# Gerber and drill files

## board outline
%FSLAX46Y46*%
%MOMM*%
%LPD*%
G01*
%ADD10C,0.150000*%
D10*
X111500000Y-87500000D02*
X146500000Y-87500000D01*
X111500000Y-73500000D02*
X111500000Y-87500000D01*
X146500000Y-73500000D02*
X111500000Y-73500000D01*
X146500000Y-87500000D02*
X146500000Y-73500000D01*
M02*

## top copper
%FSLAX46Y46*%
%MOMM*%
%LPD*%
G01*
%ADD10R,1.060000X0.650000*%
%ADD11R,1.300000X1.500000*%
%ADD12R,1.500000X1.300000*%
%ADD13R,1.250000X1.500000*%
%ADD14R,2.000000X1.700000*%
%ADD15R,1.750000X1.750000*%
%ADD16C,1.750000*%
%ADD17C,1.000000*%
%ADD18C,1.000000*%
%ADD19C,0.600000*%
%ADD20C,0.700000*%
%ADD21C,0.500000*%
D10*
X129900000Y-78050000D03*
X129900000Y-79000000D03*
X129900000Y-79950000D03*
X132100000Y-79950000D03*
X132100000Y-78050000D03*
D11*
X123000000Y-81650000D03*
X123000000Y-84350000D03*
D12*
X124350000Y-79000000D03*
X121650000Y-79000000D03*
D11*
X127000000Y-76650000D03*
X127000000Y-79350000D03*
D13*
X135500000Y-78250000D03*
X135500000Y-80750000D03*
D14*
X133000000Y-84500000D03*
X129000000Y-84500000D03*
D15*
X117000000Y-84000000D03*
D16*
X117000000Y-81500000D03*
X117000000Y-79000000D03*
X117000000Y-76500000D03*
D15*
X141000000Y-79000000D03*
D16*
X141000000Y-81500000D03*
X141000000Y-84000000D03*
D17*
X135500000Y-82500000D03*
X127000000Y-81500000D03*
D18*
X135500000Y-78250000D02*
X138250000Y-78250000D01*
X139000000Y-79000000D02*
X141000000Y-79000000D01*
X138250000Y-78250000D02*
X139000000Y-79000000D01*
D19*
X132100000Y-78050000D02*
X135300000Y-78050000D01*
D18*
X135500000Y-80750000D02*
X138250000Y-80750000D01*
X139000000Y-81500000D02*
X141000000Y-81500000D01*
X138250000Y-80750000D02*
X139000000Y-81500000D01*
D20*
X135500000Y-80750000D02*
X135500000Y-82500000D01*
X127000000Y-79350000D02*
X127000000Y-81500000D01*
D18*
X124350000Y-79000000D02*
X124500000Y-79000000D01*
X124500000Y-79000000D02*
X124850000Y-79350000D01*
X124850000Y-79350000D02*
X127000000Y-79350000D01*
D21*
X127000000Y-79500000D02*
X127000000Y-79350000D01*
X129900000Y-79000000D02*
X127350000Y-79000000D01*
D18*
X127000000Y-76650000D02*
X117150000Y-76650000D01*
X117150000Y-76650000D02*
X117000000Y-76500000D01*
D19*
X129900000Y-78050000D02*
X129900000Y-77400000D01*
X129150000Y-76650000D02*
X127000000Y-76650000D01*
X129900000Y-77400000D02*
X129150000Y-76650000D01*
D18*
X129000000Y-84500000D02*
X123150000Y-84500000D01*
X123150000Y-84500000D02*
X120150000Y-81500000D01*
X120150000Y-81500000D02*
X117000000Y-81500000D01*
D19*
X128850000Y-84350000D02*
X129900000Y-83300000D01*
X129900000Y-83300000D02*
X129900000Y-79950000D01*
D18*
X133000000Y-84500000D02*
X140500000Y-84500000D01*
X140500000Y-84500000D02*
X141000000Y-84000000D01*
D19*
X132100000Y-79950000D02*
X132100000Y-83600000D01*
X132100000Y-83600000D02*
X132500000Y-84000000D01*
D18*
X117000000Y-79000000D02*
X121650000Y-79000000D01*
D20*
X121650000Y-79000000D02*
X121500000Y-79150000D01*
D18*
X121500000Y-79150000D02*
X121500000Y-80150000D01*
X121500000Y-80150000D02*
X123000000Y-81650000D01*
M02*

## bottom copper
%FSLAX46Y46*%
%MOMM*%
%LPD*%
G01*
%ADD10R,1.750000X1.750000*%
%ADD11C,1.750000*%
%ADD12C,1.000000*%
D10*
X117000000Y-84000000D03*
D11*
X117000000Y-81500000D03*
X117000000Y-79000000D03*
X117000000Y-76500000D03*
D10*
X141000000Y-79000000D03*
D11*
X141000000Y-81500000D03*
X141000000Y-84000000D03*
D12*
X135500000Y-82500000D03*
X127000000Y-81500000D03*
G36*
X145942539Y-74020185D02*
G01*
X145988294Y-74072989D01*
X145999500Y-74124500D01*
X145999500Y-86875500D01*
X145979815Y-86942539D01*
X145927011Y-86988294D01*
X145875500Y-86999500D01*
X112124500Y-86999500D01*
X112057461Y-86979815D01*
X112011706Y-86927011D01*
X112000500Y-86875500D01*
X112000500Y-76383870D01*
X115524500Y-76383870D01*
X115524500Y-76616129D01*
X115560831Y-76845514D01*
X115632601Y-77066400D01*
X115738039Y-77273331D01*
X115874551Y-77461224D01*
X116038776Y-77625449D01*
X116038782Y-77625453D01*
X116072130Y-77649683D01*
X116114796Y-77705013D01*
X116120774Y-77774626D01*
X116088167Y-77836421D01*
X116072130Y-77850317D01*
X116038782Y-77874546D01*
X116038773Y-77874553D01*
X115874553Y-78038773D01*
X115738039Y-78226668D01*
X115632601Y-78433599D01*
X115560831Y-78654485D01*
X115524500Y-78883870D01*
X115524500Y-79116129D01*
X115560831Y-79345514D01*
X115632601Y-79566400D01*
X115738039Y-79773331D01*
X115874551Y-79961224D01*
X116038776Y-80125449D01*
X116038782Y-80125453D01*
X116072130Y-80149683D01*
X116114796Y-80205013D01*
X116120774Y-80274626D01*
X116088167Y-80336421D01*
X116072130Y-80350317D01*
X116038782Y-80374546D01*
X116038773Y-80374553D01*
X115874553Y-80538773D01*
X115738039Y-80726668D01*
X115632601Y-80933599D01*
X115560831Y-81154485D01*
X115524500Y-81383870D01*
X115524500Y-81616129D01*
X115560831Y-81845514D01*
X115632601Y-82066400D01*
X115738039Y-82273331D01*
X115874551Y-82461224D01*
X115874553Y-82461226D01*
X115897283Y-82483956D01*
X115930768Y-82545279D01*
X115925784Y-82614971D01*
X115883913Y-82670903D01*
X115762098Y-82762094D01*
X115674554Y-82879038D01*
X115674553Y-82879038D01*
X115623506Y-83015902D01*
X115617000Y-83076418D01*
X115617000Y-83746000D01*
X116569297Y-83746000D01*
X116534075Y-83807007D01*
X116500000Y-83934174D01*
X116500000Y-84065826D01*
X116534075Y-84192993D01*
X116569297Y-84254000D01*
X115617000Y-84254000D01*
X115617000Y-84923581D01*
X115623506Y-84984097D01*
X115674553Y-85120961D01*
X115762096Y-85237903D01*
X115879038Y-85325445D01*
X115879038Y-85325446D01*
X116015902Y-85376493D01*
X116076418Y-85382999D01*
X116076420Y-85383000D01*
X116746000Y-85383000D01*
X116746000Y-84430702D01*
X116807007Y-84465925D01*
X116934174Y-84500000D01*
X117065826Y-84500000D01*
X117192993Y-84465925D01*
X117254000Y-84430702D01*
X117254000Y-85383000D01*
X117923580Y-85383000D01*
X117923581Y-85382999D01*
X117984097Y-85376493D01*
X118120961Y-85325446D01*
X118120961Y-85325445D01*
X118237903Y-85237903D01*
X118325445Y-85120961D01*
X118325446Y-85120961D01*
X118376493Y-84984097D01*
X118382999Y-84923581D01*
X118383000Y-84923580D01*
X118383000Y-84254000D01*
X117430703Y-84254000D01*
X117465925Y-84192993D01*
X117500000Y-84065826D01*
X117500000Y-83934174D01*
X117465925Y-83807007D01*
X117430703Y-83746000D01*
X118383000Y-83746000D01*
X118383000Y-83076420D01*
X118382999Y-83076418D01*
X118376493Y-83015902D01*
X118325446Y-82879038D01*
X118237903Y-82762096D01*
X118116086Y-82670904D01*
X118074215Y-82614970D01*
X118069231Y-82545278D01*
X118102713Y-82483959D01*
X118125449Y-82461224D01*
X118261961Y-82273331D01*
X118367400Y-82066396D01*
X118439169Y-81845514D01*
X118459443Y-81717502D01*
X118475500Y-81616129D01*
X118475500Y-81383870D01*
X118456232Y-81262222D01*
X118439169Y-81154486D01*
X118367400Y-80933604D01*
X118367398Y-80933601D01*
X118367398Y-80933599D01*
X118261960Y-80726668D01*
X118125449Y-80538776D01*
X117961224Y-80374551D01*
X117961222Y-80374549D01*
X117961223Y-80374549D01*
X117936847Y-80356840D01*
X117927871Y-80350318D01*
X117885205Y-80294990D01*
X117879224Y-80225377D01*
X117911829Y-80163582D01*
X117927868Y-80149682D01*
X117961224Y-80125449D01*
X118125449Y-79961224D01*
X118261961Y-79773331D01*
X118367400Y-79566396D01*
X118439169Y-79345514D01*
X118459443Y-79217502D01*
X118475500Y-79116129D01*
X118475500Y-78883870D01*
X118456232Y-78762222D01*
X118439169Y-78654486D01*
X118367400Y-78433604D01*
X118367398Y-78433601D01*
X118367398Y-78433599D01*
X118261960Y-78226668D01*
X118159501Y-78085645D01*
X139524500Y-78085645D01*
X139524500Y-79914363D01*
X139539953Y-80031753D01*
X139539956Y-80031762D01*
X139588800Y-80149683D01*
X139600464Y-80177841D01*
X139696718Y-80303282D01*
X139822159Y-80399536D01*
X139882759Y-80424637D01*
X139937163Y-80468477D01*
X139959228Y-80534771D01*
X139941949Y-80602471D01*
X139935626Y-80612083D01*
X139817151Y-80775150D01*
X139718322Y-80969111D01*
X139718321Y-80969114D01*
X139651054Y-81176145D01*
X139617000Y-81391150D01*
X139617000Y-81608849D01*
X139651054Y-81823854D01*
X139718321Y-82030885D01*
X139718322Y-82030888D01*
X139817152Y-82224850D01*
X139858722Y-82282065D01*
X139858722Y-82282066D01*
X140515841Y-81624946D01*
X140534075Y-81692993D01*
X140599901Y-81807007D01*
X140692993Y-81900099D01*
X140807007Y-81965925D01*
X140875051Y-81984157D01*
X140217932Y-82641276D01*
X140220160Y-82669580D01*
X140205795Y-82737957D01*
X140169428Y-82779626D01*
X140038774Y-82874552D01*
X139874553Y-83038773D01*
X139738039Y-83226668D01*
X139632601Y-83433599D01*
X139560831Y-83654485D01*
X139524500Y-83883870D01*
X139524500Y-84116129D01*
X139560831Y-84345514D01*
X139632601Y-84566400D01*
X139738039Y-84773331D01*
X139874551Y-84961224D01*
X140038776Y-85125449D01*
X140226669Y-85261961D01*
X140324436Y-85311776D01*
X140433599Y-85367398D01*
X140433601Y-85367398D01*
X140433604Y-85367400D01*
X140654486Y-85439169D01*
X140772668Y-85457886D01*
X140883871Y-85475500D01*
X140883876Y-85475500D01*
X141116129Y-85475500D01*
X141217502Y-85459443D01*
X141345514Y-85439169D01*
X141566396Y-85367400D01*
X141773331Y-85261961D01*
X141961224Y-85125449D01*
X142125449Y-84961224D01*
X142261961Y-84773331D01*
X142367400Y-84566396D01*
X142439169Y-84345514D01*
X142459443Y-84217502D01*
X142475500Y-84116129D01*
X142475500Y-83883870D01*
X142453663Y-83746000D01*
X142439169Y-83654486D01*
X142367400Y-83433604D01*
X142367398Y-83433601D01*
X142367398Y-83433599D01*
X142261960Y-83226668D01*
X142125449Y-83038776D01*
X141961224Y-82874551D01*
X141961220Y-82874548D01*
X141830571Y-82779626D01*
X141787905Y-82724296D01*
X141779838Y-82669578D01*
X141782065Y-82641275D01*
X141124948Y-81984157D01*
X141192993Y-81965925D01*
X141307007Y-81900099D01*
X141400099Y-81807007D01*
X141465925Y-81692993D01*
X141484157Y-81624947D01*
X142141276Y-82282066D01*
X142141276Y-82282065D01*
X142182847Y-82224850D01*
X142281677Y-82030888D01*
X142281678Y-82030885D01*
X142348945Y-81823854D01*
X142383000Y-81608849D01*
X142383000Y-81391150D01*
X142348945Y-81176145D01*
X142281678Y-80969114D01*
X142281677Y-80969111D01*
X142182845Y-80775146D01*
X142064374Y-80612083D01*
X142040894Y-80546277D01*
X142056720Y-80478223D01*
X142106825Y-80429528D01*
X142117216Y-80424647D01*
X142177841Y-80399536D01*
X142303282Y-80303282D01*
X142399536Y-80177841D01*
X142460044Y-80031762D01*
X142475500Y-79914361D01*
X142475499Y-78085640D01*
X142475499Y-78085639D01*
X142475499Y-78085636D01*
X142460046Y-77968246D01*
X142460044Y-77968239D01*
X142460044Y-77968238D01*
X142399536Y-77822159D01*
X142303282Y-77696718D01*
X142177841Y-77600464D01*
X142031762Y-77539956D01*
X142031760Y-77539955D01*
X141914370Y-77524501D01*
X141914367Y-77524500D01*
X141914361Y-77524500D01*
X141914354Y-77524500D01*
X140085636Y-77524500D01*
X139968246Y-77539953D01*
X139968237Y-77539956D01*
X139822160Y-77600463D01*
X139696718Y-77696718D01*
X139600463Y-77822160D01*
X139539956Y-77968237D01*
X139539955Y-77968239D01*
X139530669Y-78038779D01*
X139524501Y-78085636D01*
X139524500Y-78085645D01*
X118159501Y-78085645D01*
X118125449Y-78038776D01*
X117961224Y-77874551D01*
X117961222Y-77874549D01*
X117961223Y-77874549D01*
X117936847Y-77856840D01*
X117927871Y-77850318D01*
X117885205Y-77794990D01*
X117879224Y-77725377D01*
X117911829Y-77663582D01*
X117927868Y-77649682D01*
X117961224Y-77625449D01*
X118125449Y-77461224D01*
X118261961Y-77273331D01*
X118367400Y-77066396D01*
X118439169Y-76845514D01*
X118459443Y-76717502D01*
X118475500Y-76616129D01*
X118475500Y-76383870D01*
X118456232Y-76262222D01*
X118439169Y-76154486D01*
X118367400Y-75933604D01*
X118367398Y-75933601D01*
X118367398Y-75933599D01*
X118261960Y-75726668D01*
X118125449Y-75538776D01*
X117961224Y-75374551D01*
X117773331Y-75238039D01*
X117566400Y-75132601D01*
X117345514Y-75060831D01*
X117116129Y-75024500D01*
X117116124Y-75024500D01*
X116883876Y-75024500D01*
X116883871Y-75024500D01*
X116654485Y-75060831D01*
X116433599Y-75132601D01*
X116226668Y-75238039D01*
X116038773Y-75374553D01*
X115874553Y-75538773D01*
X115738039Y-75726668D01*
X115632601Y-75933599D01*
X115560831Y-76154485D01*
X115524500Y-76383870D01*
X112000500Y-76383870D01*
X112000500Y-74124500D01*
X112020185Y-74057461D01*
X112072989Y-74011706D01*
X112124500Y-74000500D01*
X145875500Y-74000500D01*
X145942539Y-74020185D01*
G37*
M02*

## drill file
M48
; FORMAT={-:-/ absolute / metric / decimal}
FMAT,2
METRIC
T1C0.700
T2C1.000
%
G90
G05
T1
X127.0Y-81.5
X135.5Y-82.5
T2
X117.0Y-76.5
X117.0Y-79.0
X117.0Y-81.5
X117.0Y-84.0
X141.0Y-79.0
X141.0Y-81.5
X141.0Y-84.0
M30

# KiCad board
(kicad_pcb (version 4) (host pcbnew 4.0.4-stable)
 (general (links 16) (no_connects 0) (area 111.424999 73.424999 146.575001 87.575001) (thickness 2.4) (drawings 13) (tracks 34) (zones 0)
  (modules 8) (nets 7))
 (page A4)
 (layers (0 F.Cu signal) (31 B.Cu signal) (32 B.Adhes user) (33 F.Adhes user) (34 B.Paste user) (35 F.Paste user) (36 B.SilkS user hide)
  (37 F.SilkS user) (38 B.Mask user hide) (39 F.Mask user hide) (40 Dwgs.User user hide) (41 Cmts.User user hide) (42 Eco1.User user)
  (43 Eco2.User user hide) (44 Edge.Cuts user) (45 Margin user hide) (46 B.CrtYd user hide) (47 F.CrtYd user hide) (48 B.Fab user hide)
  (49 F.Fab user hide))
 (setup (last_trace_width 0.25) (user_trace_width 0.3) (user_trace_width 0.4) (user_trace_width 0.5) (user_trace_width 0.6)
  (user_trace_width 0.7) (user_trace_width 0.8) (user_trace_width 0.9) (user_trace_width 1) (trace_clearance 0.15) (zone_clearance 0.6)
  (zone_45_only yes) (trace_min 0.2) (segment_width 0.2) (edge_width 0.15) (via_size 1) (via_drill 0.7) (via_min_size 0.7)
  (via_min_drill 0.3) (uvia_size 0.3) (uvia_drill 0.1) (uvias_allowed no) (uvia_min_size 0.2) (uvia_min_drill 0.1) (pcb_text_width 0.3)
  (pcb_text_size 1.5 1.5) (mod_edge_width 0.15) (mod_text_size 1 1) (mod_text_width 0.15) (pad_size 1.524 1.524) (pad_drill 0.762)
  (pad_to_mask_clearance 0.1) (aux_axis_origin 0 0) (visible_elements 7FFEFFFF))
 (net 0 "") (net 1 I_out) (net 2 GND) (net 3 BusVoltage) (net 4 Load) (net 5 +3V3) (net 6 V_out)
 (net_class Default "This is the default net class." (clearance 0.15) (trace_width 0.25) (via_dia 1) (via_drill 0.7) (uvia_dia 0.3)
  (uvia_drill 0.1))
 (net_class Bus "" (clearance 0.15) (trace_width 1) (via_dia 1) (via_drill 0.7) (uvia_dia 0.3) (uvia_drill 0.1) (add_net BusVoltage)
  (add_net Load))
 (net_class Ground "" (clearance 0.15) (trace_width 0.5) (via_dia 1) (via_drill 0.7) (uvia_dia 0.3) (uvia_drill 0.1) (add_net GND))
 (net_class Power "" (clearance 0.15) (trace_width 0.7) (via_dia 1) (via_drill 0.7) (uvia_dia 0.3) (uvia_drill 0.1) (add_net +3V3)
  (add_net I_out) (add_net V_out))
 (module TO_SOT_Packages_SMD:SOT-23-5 (layer F.Cu) (at 131 79)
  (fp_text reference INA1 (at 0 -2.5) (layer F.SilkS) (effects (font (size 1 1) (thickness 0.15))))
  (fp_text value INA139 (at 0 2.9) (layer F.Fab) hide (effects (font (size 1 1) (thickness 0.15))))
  (pad 1 smd rect (at -1.1 -0.95) (size 1.06 0.65) (layers F.Cu F.Paste F.Mask) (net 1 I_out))
  (pad 2 smd rect (at -1.1 0) (size 1.06 0.65) (layers F.Cu F.Paste F.Mask) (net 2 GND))
  (pad 3 smd rect (at -1.1 0.95) (size 1.06 0.65) (layers F.Cu F.Paste F.Mask) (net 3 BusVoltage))
  (pad 4 smd rect (at 1.1 0.95) (size 1.06 0.65) (layers F.Cu F.Paste F.Mask) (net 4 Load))
  (pad 5 smd rect (at 1.1 -0.95) (size 1.06 0.65) (layers F.Cu F.Paste F.Mask) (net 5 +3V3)))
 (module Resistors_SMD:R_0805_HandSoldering (layer F.Cu) (at 123 83 270)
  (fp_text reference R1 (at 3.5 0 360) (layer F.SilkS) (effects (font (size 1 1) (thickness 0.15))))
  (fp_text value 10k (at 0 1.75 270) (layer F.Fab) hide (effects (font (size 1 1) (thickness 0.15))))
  (pad 1 smd rect (at -1.35 0 270) (size 1.5 1.3) (layers F.Cu F.Paste F.Mask) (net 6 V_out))
  (pad 2 smd rect (at 1.35 0 270) (size 1.5 1.3) (layers F.Cu F.Paste F.Mask) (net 3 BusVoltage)))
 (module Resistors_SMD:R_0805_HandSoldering (layer F.Cu) (at 123 79 180)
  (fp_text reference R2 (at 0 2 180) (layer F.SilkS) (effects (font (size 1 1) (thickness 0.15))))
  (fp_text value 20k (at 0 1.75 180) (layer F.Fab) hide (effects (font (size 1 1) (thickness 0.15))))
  (pad 1 smd rect (at -1.35 0 180) (size 1.5 1.3) (layers F.Cu F.Paste F.Mask) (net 2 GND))
  (pad 2 smd rect (at 1.35 0 180) (size 1.5 1.3) (layers F.Cu F.Paste F.Mask) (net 6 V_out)))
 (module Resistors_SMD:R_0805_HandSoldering (layer F.Cu) (at 127 78 270)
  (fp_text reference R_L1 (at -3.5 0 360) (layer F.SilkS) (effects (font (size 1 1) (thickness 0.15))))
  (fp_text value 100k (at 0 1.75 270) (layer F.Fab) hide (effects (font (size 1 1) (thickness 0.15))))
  (pad 1 smd rect (at -1.35 0 270) (size 1.5 1.3) (layers F.Cu F.Paste F.Mask) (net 1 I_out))
  (pad 2 smd rect (at 1.35 0 270) (size 1.5 1.3) (layers F.Cu F.Paste F.Mask) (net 2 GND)))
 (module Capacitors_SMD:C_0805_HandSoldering (layer F.Cu) (at 135.5 79.5 270)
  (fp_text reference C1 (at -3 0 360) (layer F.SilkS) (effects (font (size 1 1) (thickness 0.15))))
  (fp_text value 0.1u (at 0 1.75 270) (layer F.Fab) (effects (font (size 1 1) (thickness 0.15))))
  (pad 1 smd rect (at -1.25 0 270) (size 1.5 1.25) (layers F.Cu F.Paste F.Mask) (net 5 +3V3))
  (pad 2 smd rect (at 1.25 0 270) (size 1.5 1.25) (layers F.Cu F.Paste F.Mask) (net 2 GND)))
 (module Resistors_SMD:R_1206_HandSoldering (layer F.Cu) (at 131 84.5 180)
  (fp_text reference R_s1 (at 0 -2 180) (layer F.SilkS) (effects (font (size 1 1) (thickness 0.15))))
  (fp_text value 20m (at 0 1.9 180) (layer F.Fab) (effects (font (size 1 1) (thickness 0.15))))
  (pad 1 smd rect (at -2 0 180) (size 2 1.7) (layers F.Cu F.Paste F.Mask) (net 4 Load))
  (pad 2 smd rect (at 2 0 180) (size 2 1.7) (layers F.Cu F.Paste F.Mask) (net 3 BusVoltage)))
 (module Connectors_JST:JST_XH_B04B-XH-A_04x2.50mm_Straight (layer F.Cu) (at 117 84 90)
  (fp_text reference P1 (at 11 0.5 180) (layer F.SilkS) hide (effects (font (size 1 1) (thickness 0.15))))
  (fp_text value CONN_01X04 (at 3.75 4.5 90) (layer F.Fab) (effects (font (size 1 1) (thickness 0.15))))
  (pad 1 thru_hole rect (at 0 0 90) (size 1.75 1.75) (drill 1) (layers *.Cu *.Mask) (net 2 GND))
  (pad 2 thru_hole circle (at 2.5 0 90) (size 1.75 1.75) (drill 1) (layers *.Cu *.Mask) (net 3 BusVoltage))
  (pad 3 thru_hole circle (at 5 0 90) (size 1.75 1.75) (drill 1) (layers *.Cu *.Mask) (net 6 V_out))
  (pad 4 thru_hole circle (at 7.5 0 90) (size 1.75 1.75) (drill 1) (layers *.Cu *.Mask) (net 1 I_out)))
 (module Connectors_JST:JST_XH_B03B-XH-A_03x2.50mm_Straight (layer F.Cu) (at 141 79 270)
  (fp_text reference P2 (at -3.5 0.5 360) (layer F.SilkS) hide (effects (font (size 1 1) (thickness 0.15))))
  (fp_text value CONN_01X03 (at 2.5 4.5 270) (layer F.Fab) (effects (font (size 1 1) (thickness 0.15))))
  (pad 1 thru_hole rect (at 0 0 270) (size 1.75 1.75) (drill 1) (layers *.Cu *.Mask) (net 5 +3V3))
  (pad 2 thru_hole circle (at 2.5 0 270) (size 1.75 1.75) (drill 1) (layers *.Cu *.Mask) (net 2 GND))
  (pad 3 thru_hole circle (at 5 0 270) (size 1.75 1.75) (drill 1) (layers *.Cu *.Mask) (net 4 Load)))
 (gr_line (start 111.5 87.5) (end 146.5 87.5) (angle 90) (layer Edge.Cuts) (width 0.15))
 (gr_line (start 111.5 73.5) (end 111.5 87.5) (angle 90) (layer Edge.Cuts) (width 0.15))
 (gr_line (start 146.5 73.5) (end 111.5 73.5) (angle 90) (layer Edge.Cuts) (width 0.15))
 (gr_line (start 146.5 87.5) (end 146.5 73.5) (angle 90) (layer Edge.Cuts) (width 0.15))
 (segment (start 135.5 78.25) (end 138.25 78.25) (width 1) (layer F.Cu) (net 5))
 (segment (start 139 79) (end 141 79) (width 1) (layer F.Cu) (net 5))
 (segment (start 138.25 78.25) (end 139 79) (width 1) (layer F.Cu) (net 5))
 (segment (start 132.1 78.05) (end 135.3 78.05) (width 0.6) (layer F.Cu) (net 5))
 (segment (start 135.5 80.75) (end 138.25 80.75) (width 1) (layer F.Cu) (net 2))
 (segment (start 139 81.5) (end 141 81.5) (width 1) (layer F.Cu) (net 2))
 (segment (start 138.25 80.75) (end 139 81.5) (width 1) (layer F.Cu) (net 2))
 (segment (start 135.5 80.75) (end 135.5 82.5) (width 0.7) (layer F.Cu) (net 2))
 (via (at 135.5 82.5) (size 1) (drill 0.7) (layers F.Cu B.Cu) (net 2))
 (segment (start 127 79.35) (end 127 81.5) (width 0.7) (layer F.Cu) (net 2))
 (via (at 127 81.5) (size 1) (drill 0.7) (layers F.Cu B.Cu) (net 2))
 (segment (start 124.35 79) (end 124.5 79) (width 1) (layer F.Cu) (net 2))
 (segment (start 124.5 79) (end 124.85 79.35) (width 1) (layer F.Cu) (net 2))
 (segment (start 124.85 79.35) (end 127 79.35) (width 1) (layer F.Cu) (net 2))
 (segment (start 127 79.5) (end 127 79.35) (width 0.5) (layer F.Cu) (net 2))
 (segment (start 129.9 79) (end 127.35 79) (width 0.5) (layer F.Cu) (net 2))
 (segment (start 127 76.65) (end 117.15 76.65) (width 1) (layer F.Cu) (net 1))
 (segment (start 117.15 76.65) (end 117 76.5) (width 1) (layer F.Cu) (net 1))
 (segment (start 129.9 78.05) (end 129.9 77.4) (width 0.6) (layer F.Cu) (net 1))
 (segment (start 129.15 76.65) (end 127 76.65) (width 0.6) (layer F.Cu) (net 1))
 (segment (start 129.9 77.4) (end 129.15 76.65) (width 0.6) (layer F.Cu) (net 1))
 (segment (start 129 84.5) (end 123.15 84.5) (width 1) (layer F.Cu) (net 3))
 (segment (start 123.15 84.5) (end 120.15 81.5) (width 1) (layer F.Cu) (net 3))
 (segment (start 120.15 81.5) (end 117 81.5) (width 1) (layer F.Cu) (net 3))
 (segment (start 128.85 84.35) (end 129.9 83.3) (width 0.6) (layer F.Cu) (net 3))
 (segment (start 129.9 83.3) (end 129.9 79.95) (width 0.6) (layer F.Cu) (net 3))
 (segment (start 133 84.5) (end 140.5 84.5) (width 1) (layer F.Cu) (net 4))
 (segment (start 140.5 84.5) (end 141 84) (width 1) (layer F.Cu) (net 4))
 (segment (start 132.1 79.95) (end 132.1 83.6) (width 0.6) (layer F.Cu) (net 4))
 (segment (start 132.1 83.6) (end 132.5 84) (width 0.6) (layer F.Cu) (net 4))
 (segment (start 117 79) (end 121.65 79) (width 1) (layer F.Cu) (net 6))
 (segment (start 121.65 79) (end 121.5 79.15) (width 0.7) (layer F.Cu) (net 6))
 (segment (start 121.5 79.15) (end 121.5 80.15) (width 1) (layer F.Cu) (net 6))
 (segment (start 121.5 80.15) (end 123 81.65) (width 1) (layer F.Cu) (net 6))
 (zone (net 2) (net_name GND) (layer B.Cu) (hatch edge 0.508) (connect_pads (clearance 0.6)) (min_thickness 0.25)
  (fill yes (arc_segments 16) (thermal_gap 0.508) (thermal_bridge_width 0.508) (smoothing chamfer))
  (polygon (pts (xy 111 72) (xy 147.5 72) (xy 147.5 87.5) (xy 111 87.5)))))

